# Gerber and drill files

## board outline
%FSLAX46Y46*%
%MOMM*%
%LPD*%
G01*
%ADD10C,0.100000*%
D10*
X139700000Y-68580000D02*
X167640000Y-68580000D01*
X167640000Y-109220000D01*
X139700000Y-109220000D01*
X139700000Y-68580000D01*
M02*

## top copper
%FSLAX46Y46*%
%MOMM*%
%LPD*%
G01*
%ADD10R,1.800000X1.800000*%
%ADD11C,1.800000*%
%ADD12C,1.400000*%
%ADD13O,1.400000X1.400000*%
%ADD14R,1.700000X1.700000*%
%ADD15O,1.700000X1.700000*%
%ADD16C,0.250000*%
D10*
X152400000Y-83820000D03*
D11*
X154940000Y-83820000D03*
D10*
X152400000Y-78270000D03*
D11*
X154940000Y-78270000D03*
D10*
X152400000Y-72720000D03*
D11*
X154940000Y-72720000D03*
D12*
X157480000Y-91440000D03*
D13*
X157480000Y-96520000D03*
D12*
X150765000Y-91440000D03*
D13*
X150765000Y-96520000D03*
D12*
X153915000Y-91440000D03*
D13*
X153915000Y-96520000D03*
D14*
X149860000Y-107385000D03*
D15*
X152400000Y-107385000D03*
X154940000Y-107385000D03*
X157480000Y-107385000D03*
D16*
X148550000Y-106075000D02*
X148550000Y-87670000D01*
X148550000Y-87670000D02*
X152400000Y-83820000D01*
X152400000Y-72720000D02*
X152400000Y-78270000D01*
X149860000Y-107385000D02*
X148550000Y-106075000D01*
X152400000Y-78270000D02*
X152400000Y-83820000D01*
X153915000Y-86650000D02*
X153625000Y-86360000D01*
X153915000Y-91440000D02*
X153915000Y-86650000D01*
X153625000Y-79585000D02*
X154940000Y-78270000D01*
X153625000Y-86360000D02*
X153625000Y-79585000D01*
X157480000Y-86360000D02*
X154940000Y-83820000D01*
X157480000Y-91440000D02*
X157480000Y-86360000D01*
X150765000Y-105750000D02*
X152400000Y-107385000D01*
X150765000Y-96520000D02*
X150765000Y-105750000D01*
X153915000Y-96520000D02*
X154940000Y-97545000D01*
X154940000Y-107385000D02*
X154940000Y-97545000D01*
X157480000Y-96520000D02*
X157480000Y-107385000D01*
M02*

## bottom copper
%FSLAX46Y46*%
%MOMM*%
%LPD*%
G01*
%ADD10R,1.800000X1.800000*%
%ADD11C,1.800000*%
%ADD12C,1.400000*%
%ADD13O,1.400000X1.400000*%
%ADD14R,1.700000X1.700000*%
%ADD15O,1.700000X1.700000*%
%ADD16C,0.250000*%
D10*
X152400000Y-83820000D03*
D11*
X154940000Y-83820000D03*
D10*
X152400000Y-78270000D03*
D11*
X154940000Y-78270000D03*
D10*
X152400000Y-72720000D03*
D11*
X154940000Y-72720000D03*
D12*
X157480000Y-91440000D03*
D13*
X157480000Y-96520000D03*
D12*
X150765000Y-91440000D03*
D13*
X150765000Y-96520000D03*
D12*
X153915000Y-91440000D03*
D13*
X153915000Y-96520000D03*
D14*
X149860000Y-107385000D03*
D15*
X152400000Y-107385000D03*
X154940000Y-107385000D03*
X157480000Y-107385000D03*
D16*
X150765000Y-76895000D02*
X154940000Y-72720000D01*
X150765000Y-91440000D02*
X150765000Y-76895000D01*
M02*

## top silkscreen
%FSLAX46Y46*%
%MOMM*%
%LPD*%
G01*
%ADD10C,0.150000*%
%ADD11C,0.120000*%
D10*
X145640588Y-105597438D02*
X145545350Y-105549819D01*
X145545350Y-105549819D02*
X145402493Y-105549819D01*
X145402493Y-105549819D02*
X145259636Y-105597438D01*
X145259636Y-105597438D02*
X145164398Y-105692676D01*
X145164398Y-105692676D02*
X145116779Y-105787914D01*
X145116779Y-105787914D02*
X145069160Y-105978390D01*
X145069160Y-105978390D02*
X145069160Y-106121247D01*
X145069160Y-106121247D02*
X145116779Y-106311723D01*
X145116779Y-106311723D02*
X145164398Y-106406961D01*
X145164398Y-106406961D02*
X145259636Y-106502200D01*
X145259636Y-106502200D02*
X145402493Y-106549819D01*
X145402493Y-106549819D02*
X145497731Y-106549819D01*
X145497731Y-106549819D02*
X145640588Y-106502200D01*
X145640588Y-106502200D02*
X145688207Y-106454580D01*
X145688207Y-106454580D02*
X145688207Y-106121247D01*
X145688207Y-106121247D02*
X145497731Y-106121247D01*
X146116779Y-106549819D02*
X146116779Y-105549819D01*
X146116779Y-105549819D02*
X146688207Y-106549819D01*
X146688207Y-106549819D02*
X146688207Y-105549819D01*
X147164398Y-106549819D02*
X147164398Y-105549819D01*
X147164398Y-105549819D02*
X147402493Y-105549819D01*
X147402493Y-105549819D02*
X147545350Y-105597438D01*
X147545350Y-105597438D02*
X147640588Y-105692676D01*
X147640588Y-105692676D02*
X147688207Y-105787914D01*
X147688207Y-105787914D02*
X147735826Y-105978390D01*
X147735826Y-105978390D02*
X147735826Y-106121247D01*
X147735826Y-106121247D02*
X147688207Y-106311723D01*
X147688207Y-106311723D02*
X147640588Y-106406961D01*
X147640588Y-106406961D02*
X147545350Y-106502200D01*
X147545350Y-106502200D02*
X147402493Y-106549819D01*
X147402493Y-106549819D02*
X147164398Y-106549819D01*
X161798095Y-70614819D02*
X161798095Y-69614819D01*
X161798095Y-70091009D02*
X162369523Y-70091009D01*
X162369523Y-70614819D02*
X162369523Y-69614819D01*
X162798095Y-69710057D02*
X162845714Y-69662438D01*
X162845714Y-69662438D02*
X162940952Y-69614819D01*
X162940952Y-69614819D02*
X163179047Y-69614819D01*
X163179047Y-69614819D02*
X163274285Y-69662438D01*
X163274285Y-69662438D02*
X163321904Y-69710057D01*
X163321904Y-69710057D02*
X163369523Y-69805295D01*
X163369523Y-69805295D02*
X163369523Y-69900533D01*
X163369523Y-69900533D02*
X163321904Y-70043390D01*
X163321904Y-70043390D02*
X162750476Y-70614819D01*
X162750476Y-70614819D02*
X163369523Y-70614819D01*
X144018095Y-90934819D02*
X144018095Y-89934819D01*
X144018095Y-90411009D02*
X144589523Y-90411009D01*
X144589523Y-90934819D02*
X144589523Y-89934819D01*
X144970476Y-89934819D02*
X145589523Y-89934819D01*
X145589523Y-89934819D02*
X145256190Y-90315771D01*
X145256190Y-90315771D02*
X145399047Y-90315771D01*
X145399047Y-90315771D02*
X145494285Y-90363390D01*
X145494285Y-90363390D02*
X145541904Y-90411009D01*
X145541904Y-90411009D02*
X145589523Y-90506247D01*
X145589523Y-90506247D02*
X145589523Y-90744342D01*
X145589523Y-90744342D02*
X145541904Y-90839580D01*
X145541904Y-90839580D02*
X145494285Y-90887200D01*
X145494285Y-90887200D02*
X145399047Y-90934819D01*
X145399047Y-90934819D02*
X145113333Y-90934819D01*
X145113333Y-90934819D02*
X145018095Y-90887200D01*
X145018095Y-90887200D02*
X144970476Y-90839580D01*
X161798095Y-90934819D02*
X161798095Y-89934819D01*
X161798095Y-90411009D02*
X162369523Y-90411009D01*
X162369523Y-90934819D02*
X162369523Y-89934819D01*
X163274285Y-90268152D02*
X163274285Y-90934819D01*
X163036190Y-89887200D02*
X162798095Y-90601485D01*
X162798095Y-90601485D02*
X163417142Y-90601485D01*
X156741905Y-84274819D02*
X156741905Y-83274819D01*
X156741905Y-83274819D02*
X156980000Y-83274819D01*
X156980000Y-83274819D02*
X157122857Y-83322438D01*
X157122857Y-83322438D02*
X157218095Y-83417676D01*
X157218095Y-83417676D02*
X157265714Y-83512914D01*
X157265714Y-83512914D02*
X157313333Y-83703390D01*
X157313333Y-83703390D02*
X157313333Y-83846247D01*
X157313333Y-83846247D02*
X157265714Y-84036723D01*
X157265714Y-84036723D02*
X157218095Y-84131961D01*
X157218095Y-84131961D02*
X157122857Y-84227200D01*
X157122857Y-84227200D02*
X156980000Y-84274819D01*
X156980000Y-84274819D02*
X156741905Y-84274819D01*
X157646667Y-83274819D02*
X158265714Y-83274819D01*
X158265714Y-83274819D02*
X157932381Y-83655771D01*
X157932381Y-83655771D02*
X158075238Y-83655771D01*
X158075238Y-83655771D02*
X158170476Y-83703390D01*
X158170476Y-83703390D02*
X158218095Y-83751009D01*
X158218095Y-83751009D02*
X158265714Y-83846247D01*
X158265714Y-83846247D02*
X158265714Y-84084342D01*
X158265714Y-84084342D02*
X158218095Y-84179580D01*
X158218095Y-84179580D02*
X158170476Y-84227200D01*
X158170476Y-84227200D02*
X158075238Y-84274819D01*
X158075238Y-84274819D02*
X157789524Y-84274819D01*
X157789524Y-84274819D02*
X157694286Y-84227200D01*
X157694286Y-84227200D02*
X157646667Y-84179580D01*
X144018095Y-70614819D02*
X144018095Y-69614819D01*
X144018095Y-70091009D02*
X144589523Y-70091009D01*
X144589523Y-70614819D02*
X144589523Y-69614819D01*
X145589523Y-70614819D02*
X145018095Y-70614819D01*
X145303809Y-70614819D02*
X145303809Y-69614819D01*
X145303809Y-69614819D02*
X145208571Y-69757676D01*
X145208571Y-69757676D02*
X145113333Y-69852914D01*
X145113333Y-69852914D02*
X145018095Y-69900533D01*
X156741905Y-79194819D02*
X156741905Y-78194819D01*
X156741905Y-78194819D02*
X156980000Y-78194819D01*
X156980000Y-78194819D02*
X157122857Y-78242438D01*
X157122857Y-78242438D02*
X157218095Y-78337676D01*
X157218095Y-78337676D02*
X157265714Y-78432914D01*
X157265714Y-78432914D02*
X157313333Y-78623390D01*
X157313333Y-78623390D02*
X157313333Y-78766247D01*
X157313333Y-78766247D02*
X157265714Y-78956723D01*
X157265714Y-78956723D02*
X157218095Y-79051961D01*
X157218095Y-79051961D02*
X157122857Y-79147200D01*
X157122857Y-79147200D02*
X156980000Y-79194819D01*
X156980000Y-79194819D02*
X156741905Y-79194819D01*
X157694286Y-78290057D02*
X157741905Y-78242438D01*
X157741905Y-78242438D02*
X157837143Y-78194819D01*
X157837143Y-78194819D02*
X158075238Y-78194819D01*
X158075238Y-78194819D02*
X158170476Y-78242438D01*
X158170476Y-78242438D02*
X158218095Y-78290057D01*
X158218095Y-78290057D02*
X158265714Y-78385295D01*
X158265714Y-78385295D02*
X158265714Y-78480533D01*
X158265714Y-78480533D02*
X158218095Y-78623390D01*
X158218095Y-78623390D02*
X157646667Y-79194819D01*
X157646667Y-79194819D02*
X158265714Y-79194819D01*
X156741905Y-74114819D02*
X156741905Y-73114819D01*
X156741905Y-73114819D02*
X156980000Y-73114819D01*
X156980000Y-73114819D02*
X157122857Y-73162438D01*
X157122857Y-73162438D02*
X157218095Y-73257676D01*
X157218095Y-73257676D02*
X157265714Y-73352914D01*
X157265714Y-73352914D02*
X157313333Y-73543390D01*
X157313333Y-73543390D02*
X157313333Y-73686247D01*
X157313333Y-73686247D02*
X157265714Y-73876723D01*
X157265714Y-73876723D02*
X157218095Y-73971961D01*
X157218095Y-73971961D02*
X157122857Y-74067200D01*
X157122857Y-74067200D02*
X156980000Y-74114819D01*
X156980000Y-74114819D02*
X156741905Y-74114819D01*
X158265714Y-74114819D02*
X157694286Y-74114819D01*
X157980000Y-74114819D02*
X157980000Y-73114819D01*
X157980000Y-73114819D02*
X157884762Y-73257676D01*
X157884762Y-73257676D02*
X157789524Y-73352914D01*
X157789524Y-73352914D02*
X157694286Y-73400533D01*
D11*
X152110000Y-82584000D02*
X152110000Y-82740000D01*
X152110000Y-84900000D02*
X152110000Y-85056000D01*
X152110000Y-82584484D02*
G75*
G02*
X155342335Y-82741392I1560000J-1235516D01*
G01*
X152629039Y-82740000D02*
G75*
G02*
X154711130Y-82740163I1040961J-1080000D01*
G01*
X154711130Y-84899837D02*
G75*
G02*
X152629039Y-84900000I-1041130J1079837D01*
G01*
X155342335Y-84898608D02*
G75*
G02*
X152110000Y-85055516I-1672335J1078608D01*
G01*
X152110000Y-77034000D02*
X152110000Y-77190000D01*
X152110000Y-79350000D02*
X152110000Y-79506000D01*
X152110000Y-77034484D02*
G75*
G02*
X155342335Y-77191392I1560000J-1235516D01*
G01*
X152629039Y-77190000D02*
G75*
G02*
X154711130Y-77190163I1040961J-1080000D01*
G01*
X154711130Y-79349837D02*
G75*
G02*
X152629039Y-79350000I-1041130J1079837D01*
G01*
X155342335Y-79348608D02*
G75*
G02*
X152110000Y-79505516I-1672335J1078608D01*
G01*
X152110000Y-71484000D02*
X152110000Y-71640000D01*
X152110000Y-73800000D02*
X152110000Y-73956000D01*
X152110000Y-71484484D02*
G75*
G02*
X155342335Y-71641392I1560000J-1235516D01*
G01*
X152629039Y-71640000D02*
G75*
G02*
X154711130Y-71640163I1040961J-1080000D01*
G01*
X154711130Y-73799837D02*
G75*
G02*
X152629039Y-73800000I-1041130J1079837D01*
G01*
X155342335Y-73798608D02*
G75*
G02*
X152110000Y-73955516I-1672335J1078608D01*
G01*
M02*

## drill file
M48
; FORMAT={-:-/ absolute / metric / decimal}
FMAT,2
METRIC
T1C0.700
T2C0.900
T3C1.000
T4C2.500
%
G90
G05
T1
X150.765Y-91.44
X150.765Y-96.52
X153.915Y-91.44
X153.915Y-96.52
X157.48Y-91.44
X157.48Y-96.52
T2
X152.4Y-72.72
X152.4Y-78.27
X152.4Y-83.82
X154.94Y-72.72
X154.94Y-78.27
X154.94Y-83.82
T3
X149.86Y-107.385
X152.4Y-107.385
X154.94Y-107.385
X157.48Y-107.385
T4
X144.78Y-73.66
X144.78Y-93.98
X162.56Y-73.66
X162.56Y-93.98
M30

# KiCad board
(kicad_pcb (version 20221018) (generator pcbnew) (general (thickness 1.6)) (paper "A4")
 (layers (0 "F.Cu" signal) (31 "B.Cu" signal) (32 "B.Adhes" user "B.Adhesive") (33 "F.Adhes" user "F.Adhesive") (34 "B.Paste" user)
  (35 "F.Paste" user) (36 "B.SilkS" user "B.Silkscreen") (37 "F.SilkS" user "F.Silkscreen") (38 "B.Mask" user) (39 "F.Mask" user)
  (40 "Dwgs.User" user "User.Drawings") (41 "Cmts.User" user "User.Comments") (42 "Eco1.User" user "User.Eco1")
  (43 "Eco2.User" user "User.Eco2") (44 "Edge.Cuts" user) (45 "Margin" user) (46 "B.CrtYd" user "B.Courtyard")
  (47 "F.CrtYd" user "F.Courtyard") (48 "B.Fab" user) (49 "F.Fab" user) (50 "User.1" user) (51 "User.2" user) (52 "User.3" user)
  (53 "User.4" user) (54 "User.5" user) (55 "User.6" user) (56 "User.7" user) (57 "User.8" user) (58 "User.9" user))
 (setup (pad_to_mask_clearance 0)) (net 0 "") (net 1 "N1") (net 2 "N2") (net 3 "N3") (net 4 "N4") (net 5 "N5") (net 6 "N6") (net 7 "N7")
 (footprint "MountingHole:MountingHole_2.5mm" (layer "F.Cu") (at 162.56 73.66)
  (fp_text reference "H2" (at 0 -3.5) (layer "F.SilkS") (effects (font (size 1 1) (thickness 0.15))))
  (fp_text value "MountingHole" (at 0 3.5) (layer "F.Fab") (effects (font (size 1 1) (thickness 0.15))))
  (pad "" np_thru_hole circle (at 0 0) (size 2.5 2.5) (drill 2.5) (layers "*.Cu" "*.Mask")))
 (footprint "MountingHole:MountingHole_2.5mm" (layer "F.Cu") (at 144.78 93.98)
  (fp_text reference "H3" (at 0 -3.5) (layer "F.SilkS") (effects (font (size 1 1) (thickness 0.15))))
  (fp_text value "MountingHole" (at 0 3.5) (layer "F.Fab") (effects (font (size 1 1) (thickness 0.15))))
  (pad "" np_thru_hole circle (at 0 0) (size 2.5 2.5) (drill 2.5) (layers "*.Cu" "*.Mask")))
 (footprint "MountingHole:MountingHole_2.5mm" (layer "F.Cu") (at 162.56 93.98)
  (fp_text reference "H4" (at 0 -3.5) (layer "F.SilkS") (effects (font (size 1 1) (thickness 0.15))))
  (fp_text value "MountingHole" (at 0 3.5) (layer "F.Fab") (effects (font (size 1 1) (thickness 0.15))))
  (pad "" np_thru_hole circle (at 0 0) (size 2.5 2.5) (drill 2.5) (layers "*.Cu" "*.Mask")))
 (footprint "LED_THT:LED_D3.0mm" (layer "F.Cu") (at 152.4 83.82)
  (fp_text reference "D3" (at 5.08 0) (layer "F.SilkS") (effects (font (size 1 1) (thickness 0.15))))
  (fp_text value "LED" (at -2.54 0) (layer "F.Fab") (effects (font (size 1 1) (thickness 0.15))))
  (fp_line (start -0.29 -1.236) (end -0.29 -1.08) (stroke (width 0.12) (type solid)) (layer "F.SilkS"))
  (fp_line (start -0.29 1.08) (end -0.29 1.236) (stroke (width 0.12) (type solid)) (layer "F.SilkS"))
  (fp_arc (start -0.29 -1.235516) (mid 1.366487 -1.987659) (end 2.942335 -1.078608) (stroke (width 0.12) (type solid)) (layer "F.SilkS"))
  (fp_arc (start 0.229039 -1.08) (mid 1.270117 -1.5) (end 2.31113 -1.079837) (stroke (width 0.12) (type solid)) (layer "F.SilkS"))
  (fp_arc (start 2.31113 1.079837) (mid 1.270117 1.5) (end 0.229039 1.08) (stroke (width 0.12) (type solid)) (layer "F.SilkS"))
  (fp_arc (start 2.942335 1.078608) (mid 1.366487 1.987659) (end -0.29 1.235516) (stroke (width 0.12) (type solid)) (layer "F.SilkS"))
  (pad "1" thru_hole rect (at 0 0) (size 1.8 1.8) (drill 0.9) (layers "*.Cu" "*.Mask") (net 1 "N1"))
  (pad "2" thru_hole circle (at 2.54 0) (size 1.8 1.8) (drill 0.9) (layers "*.Cu" "*.Mask") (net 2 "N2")))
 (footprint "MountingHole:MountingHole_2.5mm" (layer "F.Cu") (at 144.78 73.66)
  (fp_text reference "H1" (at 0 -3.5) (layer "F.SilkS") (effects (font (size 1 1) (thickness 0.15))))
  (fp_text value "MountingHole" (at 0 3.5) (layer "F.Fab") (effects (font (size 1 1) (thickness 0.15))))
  (pad "" np_thru_hole circle (at 0 0) (size 2.5 2.5) (drill 2.5) (layers "*.Cu" "*.Mask")))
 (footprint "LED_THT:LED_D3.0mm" (layer "F.Cu") (at 152.4 78.27)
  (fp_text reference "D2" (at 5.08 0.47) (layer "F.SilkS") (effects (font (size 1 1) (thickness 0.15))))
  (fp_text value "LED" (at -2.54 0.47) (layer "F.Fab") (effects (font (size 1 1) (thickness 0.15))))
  (fp_line (start -0.29 -1.236) (end -0.29 -1.08) (stroke (width 0.12) (type solid)) (layer "F.SilkS"))
  (fp_line (start -0.29 1.08) (end -0.29 1.236) (stroke (width 0.12) (type solid)) (layer "F.SilkS"))
  (fp_arc (start -0.29 -1.235516) (mid 1.366487 -1.987659) (end 2.942335 -1.078608) (stroke (width 0.12) (type solid)) (layer "F.SilkS"))
  (fp_arc (start 0.229039 -1.08) (mid 1.270117 -1.5) (end 2.31113 -1.079837) (stroke (width 0.12) (type solid)) (layer "F.SilkS"))
  (fp_arc (start 2.31113 1.079837) (mid 1.270117 1.5) (end 0.229039 1.08) (stroke (width 0.12) (type solid)) (layer "F.SilkS"))
  (fp_arc (start 2.942335 1.078608) (mid 1.366487 1.987659) (end -0.29 1.235516) (stroke (width 0.12) (type solid)) (layer "F.SilkS"))
  (pad "1" thru_hole rect (at 0 0) (size 1.8 1.8) (drill 0.9) (layers "*.Cu" "*.Mask") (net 1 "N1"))
  (pad "2" thru_hole circle (at 2.54 0) (size 1.8 1.8) (drill 0.9) (layers "*.Cu" "*.Mask") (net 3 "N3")))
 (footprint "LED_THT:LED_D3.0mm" (layer "F.Cu") (at 152.4 72.72)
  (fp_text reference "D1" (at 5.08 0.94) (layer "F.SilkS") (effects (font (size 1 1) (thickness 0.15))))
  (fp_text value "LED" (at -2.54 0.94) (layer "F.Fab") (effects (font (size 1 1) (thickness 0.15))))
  (fp_line (start -0.29 -1.236) (end -0.29 -1.08) (stroke (width 0.12) (type solid)) (layer "F.SilkS"))
  (fp_line (start -0.29 1.08) (end -0.29 1.236) (stroke (width 0.12) (type solid)) (layer "F.SilkS"))
  (fp_arc (start -0.29 -1.235516) (mid 1.366487 -1.987659) (end 2.942335 -1.078608) (stroke (width 0.12) (type solid)) (layer "F.SilkS"))
  (fp_arc (start 0.229039 -1.08) (mid 1.270117 -1.5) (end 2.31113 -1.079837) (stroke (width 0.12) (type solid)) (layer "F.SilkS"))
  (fp_arc (start 2.31113 1.079837) (mid 1.270117 1.5) (end 0.229039 1.08) (stroke (width 0.12) (type solid)) (layer "F.SilkS"))
  (fp_arc (start 2.942335 1.078608) (mid 1.366487 1.987659) (end -0.29 1.235516) (stroke (width 0.12) (type solid)) (layer "F.SilkS"))
  (pad "1" thru_hole rect (at 0 0) (size 1.8 1.8) (drill 0.9) (layers "*.Cu" "*.Mask") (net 1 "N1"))
  (pad "2" thru_hole circle (at 2.54 0) (size 1.8 1.8) (drill 0.9) (layers "*.Cu" "*.Mask") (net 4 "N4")))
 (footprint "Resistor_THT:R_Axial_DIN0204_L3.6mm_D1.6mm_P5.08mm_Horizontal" (layer "B.Cu") (at 157.48 91.44 -90)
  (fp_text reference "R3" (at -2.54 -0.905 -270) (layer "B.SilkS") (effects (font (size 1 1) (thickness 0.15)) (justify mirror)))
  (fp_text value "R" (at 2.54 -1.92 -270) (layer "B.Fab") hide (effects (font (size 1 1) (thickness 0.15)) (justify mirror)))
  (pad "1" thru_hole circle (at 0 0 270) (size 1.4 1.4) (drill 0.7) (layers "*.Cu" "*.Mask") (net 2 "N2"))
  (pad "2" thru_hole oval (at 5.08 0 270) (size 1.4 1.4) (drill 0.7) (layers "*.Cu" "*.Mask") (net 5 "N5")))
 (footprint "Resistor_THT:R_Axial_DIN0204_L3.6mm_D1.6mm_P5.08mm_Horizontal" (layer "B.Cu") (at 150.765 91.44 -90)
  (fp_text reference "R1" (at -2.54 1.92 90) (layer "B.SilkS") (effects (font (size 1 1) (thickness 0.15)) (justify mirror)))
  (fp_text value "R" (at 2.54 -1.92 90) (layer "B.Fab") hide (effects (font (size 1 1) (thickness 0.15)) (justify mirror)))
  (pad "1" thru_hole circle (at 0 0 270) (size 1.4 1.4) (drill 0.7) (layers "*.Cu" "*.Mask") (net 4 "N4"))
  (pad "2" thru_hole oval (at 5.08 0 270) (size 1.4 1.4) (drill 0.7) (layers "*.Cu" "*.Mask") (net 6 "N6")))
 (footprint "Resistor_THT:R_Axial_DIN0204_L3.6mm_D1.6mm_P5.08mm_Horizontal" (layer "B.Cu") (at 153.915 91.44 -90)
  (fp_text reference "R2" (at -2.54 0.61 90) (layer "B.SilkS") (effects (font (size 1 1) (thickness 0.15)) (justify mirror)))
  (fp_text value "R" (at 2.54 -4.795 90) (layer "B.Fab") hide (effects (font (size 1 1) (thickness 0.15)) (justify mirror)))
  (pad "1" thru_hole circle (at 0 0 270) (size 1.4 1.4) (drill 0.7) (layers "*.Cu" "*.Mask") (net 3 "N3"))
  (pad "2" thru_hole oval (at 5.08 0 270) (size 1.4 1.4) (drill 0.7) (layers "*.Cu" "*.Mask") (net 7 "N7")))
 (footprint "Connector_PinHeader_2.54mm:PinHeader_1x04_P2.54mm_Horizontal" (layer "B.Cu") (at 149.86 107.385 -90)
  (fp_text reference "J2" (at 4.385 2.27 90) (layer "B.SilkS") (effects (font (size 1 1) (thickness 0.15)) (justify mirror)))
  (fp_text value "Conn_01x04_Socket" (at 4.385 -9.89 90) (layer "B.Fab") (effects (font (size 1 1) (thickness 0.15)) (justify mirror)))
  (pad "1" thru_hole rect (at 0 0 270) (size 1.7 1.7) (drill 1) (layers "*.Cu" "*.Mask") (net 1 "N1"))
  (pad "2" thru_hole oval (at 0 -2.54 270) (size 1.7 1.7) (drill 1) (layers "*.Cu" "*.Mask") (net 6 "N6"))
  (pad "3" thru_hole oval (at 0 -5.08 270) (size 1.7 1.7) (drill 1) (layers "*.Cu" "*.Mask") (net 7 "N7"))
  (pad "4" thru_hole oval (at 0 -7.62 270) (size 1.7 1.7) (drill 1) (layers "*.Cu" "*.Mask") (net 5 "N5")))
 (gr_rect (start 139.7 68.58) (end 167.64 109.22) (stroke (width 0.1) (type default)) (fill none) (layer "Edge.Cuts"))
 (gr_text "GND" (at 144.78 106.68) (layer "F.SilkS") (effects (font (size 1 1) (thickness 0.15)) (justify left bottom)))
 (segment (start 148.55 106.075) (end 148.55 87.67) (width 0.25) (layer "F.Cu") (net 1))
 (segment (start 148.55 87.67) (end 152.4 83.82) (width 0.25) (layer "F.Cu") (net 1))
 (segment (start 152.4 72.72) (end 152.4 78.27) (width 0.25) (layer "F.Cu") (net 1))
 (segment (start 149.86 107.385) (end 148.55 106.075) (width 0.25) (layer "F.Cu") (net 1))
 (segment (start 152.4 78.27) (end 152.4 83.82) (width 0.25) (layer "F.Cu") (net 1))
 (segment (start 150.765 76.895) (end 154.94 72.72) (width 0.25) (layer "B.Cu") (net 4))
 (segment (start 150.765 91.44) (end 150.765 76.895) (width 0.25) (layer "B.Cu") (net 4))
 (segment (start 153.915 86.65) (end 153.625 86.36) (width 0.25) (layer "F.Cu") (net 3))
 (segment (start 153.915 91.44) (end 153.915 86.65) (width 0.25) (layer "F.Cu") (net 3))
 (segment (start 153.625 79.585) (end 154.94 78.27) (width 0.25) (layer "F.Cu") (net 3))
 (segment (start 153.625 86.36) (end 153.625 79.585) (width 0.25) (layer "F.Cu") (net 3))
 (segment (start 157.48 86.36) (end 154.94 83.82) (width 0.25) (layer "F.Cu") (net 2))
 (segment (start 157.48 91.44) (end 157.48 86.36) (width 0.25) (layer "F.Cu") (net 2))
 (segment (start 150.765 105.75) (end 152.4 107.385) (width 0.25) (layer "F.Cu") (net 6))
 (segment (start 150.765 96.52) (end 150.765 105.75) (width 0.25) (layer "F.Cu") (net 6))
 (segment (start 153.915 96.52) (end 154.94 97.545) (width 0.25) (layer "F.Cu") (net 7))
 (segment (start 154.94 107.385) (end 154.94 97.545) (width 0.25) (layer "F.Cu") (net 7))
 (segment (start 157.48 96.52) (end 157.48 107.385) (width 0.25) (layer "F.Cu") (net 5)))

